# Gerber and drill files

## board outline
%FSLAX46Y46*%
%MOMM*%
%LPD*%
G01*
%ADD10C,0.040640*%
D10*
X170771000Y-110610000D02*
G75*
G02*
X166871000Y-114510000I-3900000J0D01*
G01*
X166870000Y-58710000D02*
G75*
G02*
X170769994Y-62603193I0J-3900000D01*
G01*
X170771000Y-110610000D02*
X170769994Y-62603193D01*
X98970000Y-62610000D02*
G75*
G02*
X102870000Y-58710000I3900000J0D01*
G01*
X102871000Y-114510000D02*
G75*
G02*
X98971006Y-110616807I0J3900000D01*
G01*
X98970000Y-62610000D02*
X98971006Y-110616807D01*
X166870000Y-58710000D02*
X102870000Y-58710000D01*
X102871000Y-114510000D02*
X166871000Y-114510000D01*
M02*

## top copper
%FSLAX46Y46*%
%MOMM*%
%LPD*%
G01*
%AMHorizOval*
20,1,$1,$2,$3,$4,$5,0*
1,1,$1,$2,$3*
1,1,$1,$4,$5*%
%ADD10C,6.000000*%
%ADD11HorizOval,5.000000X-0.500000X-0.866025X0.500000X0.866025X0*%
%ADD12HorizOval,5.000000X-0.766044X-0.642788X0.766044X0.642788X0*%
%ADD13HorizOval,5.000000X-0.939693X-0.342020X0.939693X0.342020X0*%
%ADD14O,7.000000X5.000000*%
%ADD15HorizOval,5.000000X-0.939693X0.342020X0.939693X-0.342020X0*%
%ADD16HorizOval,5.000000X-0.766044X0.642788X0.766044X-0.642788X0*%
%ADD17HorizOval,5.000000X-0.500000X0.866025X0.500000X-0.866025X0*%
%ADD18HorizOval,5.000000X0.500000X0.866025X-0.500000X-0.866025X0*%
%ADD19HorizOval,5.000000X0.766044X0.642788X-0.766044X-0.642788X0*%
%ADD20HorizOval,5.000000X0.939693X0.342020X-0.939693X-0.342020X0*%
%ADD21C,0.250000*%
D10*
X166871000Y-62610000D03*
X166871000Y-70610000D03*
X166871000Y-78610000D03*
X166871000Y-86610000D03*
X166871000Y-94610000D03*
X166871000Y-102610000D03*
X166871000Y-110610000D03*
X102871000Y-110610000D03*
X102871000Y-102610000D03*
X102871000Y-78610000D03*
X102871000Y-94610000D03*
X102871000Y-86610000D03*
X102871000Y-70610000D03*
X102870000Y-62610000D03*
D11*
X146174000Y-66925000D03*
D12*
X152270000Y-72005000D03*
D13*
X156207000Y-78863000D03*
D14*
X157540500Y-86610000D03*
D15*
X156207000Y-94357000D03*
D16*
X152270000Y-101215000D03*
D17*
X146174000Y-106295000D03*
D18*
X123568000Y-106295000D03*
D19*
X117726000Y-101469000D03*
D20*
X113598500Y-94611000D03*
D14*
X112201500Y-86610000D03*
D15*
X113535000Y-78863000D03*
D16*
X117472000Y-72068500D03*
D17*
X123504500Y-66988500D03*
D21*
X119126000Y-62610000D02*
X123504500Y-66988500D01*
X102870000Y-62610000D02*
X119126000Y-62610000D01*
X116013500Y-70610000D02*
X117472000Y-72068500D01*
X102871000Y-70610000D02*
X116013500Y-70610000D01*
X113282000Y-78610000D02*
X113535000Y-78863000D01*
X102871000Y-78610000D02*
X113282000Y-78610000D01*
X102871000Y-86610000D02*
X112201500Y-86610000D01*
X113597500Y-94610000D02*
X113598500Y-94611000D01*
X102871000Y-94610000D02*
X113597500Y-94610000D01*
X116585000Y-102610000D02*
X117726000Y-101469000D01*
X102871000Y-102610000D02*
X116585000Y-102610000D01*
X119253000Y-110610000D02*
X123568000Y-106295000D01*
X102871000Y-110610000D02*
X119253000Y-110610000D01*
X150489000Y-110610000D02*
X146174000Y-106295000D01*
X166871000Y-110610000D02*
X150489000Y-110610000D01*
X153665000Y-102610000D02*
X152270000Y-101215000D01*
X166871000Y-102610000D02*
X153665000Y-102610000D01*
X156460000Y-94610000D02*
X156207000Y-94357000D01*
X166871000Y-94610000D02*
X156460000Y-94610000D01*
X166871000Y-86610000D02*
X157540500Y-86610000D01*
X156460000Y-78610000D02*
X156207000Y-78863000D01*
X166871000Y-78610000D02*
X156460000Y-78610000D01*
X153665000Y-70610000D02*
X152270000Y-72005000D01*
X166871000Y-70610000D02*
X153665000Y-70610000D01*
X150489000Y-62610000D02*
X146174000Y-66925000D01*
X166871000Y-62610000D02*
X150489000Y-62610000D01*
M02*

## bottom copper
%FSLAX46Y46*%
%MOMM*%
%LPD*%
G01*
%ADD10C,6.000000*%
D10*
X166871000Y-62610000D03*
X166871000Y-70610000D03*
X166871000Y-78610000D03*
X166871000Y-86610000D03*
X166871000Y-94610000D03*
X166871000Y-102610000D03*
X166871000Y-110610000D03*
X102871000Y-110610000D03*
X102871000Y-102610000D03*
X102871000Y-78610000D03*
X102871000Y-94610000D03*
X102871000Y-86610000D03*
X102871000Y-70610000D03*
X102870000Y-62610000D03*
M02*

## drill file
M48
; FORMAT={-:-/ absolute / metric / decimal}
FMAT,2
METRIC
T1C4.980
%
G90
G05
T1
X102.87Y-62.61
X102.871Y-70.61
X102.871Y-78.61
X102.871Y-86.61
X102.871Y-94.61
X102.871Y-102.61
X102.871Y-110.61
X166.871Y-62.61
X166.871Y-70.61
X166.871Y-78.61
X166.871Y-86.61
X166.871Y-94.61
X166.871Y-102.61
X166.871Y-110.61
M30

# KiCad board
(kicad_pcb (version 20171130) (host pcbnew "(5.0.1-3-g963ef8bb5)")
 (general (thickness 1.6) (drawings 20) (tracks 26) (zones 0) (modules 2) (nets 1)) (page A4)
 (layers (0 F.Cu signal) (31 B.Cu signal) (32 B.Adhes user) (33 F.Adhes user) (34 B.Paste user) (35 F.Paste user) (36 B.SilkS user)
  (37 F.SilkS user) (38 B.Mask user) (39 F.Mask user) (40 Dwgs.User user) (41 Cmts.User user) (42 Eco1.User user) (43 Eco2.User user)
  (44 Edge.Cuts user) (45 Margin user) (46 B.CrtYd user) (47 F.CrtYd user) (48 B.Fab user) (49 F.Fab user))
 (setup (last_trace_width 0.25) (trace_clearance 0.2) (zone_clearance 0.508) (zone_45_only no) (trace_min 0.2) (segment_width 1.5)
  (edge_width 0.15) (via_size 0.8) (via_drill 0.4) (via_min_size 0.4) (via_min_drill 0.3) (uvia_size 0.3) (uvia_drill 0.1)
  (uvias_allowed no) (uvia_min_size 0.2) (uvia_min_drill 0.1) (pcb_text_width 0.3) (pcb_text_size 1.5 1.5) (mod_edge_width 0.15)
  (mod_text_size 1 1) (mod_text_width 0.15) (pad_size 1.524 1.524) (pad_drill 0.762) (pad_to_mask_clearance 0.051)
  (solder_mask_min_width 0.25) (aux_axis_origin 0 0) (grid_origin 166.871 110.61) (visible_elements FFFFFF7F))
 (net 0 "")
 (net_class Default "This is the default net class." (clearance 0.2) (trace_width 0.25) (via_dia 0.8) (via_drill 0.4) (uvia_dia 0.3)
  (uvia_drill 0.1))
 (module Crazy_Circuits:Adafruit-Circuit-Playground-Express (layer F.Cu) (at 102.87 54.61)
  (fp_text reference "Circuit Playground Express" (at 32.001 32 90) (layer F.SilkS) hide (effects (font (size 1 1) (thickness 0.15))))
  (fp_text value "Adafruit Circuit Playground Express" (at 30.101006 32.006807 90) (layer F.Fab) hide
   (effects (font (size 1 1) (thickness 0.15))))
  (fp_arc (start 64.001 56) (end 67.901 56) (angle 90) (layer Edge.Cuts) (width 0.04064))
  (fp_arc (start 64 8) (end 64 4.1) (angle 89.89999678) (layer Edge.Cuts) (width 0.04064))
  (fp_line (start 67.901 56) (end 67.899994 7.993193) (layer Edge.Cuts) (width 0.04064))
  (fp_arc (start 0 8) (end -3.9 8) (angle 90) (layer Edge.Cuts) (width 0.04064))
  (fp_arc (start 0.001 56) (end 0.001 59.9) (angle 89.89999678) (layer Edge.Cuts) (width 0.04064))
  (fp_line (start -3.9 8) (end -3.898994 56.006807) (layer Edge.Cuts) (width 0.04064))
  (fp_line (start 64 4.1) (end 0 4.1) (layer Edge.Cuts) (width 0.04064))
  (fp_line (start 0.001 59.9) (end 64.001 59.9) (layer Edge.Cuts) (width 0.04064))
  (pad GND thru_hole circle (at 64.001 8 90) (size 6 6) (drill 4.98) (layers *.Cu *.Mask))
  (pad A7 thru_hole circle (at 64.001 16 90) (size 6 6) (drill 4.98) (layers *.Cu *.Mask))
  (pad A6 thru_hole circle (at 64.001 24 90) (size 6 6) (drill 4.98) (layers *.Cu *.Mask))
  (pad 3.3V thru_hole circle (at 64.001 32 90) (size 6 6) (drill 4.98) (layers *.Cu *.Mask))
  (pad A5 thru_hole circle (at 64.001 40 90) (size 6 6) (drill 4.98) (layers *.Cu *.Mask))
  (pad A4 thru_hole circle (at 64.001 48 90) (size 6 6) (drill 4.98) (layers *.Cu *.Mask))
  (pad GND thru_hole circle (at 64.001 56 90) (size 6 6) (drill 4.98) (layers *.Cu *.Mask))
  (pad 3.3V thru_hole circle (at 0.001 56 90) (size 6 6) (drill 4.98) (layers *.Cu *.Mask))
  (pad A3 thru_hole circle (at 0.001 48 90) (size 6 6) (drill 4.98) (layers *.Cu *.Mask))
  (pad A1 thru_hole circle (at 0.001 24 90) (size 6 6) (drill 4.98) (layers *.Cu *.Mask))
  (pad A2 thru_hole circle (at 0.001 40 90) (size 6 6) (drill 4.98) (layers *.Cu *.Mask))
  (pad GND thru_hole circle (at 0.001 32 90) (size 6 6) (drill 4.98) (layers *.Cu *.Mask))
  (pad A0 thru_hole circle (at 0.001 16 90) (size 6 6) (drill 4.98) (layers *.Cu *.Mask))
  (pad VOUT thru_hole circle (at 0 8 90) (size 6 6) (drill 4.98) (layers *.Cu *.Mask)))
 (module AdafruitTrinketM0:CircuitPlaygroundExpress (layer F.Cu) (at 134.871 86.61)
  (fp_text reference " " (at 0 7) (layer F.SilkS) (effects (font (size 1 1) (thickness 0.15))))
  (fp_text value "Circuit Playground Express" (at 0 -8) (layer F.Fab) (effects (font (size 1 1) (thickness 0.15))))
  (pad 14 smd oval (at 11.303 -19.685 330) (size 5 7) (layers F.Cu F.Paste F.Mask))
  (pad 13 smd oval (at 17.399 -14.605 310) (size 5 7) (layers F.Cu F.Paste F.Mask))
  (pad 12 smd oval (at 21.336 -7.747 290) (size 5 7) (layers F.Cu F.Paste F.Mask))
  (pad 11 smd oval (at 22.6695 0 270) (size 5 7) (layers F.Cu F.Paste F.Mask))
  (pad 10 smd oval (at 21.336 7.747 250) (size 5 7) (layers F.Cu F.Paste F.Mask))
  (pad 9 smd oval (at 17.399 14.605 230) (size 5 7) (layers F.Cu F.Paste F.Mask))
  (pad 8 smd oval (at 11.303 19.685 210) (size 5 7) (layers F.Cu F.Paste F.Mask))
  (pad 7 smd oval (at -11.303 19.685 150) (size 5 7) (layers F.Cu F.Paste F.Mask))
  (pad 6 smd oval (at -17.145 14.859 130) (size 5 7) (layers F.Cu F.Paste F.Mask))
  (pad 5 smd oval (at -21.2725 8.001 110) (size 5 7) (layers F.Cu F.Paste F.Mask))
  (pad 4 smd oval (at -22.6695 0 90) (size 5 7) (layers F.Cu F.Paste F.Mask))
  (pad 3 smd oval (at -21.336 -7.747 70) (size 5 7) (layers F.Cu F.Paste F.Mask))
  (pad 2 smd oval (at -17.399 -14.5415 50) (size 5 7) (layers F.Cu F.Paste F.Mask))
  (pad 1 smd oval (at -11.3665 -19.6215 30) (size 5 7) (layers F.Cu F.Paste F.Mask)))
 (segment (start 119.126 62.61) (end 123.5045 66.9885) (width 0.25) (layer F.Cu) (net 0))
 (segment (start 102.87 62.61) (end 119.126 62.61) (width 0.25) (layer F.Cu) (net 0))
 (segment (start 116.0135 70.61) (end 117.472 72.0685) (width 0.25) (layer F.Cu) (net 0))
 (segment (start 102.871 70.61) (end 116.0135 70.61) (width 0.25) (layer F.Cu) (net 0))
 (segment (start 113.282 78.61) (end 113.535 78.863) (width 0.25) (layer F.Cu) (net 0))
 (segment (start 102.871 78.61) (end 113.282 78.61) (width 0.25) (layer F.Cu) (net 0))
 (segment (start 102.871 86.61) (end 112.2015 86.61) (width 0.25) (layer F.Cu) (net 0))
 (segment (start 113.5975 94.61) (end 113.5985 94.611) (width 0.25) (layer F.Cu) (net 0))
 (segment (start 102.871 94.61) (end 113.5975 94.61) (width 0.25) (layer F.Cu) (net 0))
 (segment (start 116.585 102.61) (end 117.726 101.469) (width 0.25) (layer F.Cu) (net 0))
 (segment (start 102.871 102.61) (end 116.585 102.61) (width 0.25) (layer F.Cu) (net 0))
 (segment (start 119.253 110.61) (end 123.568 106.295) (width 0.25) (layer F.Cu) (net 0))
 (segment (start 102.871 110.61) (end 119.253 110.61) (width 0.25) (layer F.Cu) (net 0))
 (segment (start 150.489 110.61) (end 146.174 106.295) (width 0.25) (layer F.Cu) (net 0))
 (segment (start 166.871 110.61) (end 150.489 110.61) (width 0.25) (layer F.Cu) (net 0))
 (segment (start 153.665 102.61) (end 152.27 101.215) (width 0.25) (layer F.Cu) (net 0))
 (segment (start 166.871 102.61) (end 153.665 102.61) (width 0.25) (layer F.Cu) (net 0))
 (segment (start 156.46 94.61) (end 156.207 94.357) (width 0.25) (layer F.Cu) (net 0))
 (segment (start 166.871 94.61) (end 156.46 94.61) (width 0.25) (layer F.Cu) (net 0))
 (segment (start 166.871 86.61) (end 157.5405 86.61) (width 0.25) (layer F.Cu) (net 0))
 (segment (start 156.46 78.61) (end 156.207 78.863) (width 0.25) (layer F.Cu) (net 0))
 (segment (start 166.871 78.61) (end 156.46 78.61) (width 0.25) (layer F.Cu) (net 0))
 (segment (start 153.665 70.61) (end 152.27 72.005) (width 0.25) (layer F.Cu) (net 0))
 (segment (start 166.871 70.61) (end 153.665 70.61) (width 0.25) (layer F.Cu) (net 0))
 (segment (start 150.489 62.61) (end 146.174 66.925) (width 0.25) (layer F.Cu) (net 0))
 (segment (start 166.871 62.61) (end 150.489 62.61) (width 0.25) (layer F.Cu) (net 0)))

